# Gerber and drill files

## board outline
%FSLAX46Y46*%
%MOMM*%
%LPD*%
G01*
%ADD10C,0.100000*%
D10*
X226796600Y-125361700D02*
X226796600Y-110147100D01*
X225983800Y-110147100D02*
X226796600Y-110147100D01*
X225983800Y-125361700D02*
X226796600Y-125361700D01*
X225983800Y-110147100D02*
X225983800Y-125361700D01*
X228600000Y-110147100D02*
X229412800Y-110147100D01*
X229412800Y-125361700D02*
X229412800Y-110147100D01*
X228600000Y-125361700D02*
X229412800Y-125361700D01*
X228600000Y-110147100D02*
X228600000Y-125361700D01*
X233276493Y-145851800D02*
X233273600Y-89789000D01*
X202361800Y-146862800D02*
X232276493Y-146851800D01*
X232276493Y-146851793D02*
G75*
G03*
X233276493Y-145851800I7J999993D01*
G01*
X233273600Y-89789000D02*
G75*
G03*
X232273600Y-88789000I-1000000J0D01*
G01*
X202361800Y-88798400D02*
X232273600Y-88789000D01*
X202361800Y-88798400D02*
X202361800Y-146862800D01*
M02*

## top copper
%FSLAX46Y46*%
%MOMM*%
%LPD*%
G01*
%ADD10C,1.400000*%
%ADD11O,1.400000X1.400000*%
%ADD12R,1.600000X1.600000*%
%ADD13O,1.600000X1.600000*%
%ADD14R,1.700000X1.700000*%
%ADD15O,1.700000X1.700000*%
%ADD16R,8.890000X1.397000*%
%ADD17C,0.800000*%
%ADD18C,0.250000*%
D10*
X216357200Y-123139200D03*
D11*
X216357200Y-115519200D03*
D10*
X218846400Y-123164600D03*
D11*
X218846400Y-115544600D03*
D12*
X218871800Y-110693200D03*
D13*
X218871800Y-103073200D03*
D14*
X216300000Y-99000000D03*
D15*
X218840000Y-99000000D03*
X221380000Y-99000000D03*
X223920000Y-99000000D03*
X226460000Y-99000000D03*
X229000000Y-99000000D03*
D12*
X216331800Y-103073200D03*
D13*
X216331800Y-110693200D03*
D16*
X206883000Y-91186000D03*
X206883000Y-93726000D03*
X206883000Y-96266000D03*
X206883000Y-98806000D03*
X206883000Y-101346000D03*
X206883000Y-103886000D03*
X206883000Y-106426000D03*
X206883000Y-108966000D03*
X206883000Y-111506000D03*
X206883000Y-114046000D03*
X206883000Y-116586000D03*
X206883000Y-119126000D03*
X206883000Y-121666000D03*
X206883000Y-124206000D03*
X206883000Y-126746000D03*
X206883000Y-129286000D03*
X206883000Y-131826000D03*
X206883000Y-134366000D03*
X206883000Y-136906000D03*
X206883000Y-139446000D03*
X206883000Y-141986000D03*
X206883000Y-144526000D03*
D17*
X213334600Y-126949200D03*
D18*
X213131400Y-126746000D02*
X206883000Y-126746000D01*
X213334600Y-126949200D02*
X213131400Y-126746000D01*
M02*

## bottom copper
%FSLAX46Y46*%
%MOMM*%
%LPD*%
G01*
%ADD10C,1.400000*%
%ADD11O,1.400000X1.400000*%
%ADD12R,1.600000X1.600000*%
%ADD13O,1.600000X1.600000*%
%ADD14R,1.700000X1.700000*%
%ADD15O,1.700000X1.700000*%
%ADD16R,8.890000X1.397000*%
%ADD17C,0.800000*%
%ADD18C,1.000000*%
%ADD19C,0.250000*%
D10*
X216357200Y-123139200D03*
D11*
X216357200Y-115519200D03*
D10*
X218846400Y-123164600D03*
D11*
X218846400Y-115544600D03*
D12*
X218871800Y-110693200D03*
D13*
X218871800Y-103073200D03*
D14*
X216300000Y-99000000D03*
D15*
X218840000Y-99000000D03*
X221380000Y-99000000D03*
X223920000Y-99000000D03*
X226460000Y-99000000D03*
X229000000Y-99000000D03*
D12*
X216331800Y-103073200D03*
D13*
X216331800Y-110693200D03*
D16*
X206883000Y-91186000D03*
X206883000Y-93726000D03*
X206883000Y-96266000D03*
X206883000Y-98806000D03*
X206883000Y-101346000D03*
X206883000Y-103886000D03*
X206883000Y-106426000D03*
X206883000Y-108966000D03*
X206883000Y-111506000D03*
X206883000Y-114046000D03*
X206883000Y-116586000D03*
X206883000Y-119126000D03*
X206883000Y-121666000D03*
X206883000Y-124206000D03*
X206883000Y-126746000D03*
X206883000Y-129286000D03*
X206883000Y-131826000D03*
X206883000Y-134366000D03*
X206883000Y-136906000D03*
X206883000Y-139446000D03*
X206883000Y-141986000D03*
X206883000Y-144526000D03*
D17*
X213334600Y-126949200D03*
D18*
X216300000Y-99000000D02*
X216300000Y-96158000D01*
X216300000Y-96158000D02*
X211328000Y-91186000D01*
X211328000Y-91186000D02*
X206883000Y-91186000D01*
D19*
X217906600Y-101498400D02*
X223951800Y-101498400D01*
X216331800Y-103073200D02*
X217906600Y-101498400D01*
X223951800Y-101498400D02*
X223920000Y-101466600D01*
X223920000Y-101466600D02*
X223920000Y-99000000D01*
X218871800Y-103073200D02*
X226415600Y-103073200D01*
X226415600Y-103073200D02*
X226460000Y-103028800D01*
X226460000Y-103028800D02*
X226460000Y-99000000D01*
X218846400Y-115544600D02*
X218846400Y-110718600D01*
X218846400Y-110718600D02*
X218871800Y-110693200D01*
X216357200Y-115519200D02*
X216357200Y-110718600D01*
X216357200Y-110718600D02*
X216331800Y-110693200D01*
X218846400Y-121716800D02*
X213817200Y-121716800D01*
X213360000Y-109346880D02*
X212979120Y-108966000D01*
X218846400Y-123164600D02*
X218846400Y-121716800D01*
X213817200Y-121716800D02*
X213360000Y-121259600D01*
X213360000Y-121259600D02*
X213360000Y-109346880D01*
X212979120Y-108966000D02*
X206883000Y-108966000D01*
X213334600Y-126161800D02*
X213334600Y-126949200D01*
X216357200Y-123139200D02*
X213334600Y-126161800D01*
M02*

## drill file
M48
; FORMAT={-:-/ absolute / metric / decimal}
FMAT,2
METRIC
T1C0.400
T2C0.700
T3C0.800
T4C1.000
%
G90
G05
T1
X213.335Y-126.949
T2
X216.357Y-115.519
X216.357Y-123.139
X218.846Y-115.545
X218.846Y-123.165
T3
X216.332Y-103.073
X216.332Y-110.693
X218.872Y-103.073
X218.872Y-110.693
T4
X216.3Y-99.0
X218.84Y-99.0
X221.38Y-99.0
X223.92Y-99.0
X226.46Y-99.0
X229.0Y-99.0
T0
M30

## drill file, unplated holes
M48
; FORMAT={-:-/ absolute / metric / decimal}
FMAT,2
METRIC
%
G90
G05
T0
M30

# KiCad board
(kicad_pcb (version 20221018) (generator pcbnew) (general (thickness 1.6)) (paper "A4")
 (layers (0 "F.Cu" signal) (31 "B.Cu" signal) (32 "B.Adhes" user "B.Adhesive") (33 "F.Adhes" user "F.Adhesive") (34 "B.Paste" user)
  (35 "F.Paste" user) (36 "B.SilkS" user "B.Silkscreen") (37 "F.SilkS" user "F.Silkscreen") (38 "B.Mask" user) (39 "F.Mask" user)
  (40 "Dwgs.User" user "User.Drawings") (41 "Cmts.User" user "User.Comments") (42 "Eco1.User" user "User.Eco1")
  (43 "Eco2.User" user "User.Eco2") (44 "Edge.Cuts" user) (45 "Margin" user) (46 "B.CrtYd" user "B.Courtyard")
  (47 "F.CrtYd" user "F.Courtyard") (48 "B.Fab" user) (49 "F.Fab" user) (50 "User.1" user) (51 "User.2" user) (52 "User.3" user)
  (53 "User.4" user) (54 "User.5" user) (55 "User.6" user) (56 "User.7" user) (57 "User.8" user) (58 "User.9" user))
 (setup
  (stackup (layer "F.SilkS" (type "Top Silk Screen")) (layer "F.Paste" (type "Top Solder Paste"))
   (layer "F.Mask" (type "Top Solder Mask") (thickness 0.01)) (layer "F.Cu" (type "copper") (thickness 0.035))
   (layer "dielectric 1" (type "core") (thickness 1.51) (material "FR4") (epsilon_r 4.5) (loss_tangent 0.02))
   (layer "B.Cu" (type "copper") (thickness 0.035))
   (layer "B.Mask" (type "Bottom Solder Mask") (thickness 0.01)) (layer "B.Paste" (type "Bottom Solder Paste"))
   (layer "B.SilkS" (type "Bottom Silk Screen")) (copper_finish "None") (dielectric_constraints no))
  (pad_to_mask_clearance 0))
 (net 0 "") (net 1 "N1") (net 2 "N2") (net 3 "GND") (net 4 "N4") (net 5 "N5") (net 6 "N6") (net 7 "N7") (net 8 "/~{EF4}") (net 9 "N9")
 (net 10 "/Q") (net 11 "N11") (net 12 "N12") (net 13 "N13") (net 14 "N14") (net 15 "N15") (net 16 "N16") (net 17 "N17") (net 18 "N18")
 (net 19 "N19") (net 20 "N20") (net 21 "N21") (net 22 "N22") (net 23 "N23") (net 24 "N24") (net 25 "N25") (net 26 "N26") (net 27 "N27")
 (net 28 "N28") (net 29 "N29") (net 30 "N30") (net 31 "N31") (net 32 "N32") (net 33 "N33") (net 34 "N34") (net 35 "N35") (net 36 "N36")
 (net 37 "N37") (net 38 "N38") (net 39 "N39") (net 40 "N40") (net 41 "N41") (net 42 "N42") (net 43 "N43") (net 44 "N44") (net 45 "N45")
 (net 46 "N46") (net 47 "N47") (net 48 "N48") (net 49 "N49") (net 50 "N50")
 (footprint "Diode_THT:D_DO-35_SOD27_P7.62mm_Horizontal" (layer "F.Cu") (at 218.8718 110.6932 90)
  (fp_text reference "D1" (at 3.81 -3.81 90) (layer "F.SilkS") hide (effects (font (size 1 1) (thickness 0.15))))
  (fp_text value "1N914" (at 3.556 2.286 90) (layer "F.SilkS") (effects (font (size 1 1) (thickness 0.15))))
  (pad "1" thru_hole rect (at 0 0 90) (size 1.6 1.6) (drill 0.8) (layers "*.Cu" "*.Mask") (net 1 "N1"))
  (pad "2" thru_hole oval (at 7.62 0 90) (size 1.6 1.6) (drill 0.8) (layers "*.Cu" "*.Mask") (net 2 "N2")))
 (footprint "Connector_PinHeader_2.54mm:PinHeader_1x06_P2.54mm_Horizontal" (layer "F.Cu") (at 216.3 99 90)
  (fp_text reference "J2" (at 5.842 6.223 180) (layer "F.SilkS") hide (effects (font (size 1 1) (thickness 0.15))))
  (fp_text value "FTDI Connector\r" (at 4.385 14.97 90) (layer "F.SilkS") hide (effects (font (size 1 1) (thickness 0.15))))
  (pad "1" thru_hole rect (at 0 0 90) (size 1.7 1.7) (drill 1) (layers "*.Cu" "*.Mask") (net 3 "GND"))
  (pad "2" thru_hole oval (at 0 2.54 90) (size 1.7 1.7) (drill 1) (layers "*.Cu" "*.Mask") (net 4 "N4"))
  (pad "3" thru_hole oval (at 0 5.08 90) (size 1.7 1.7) (drill 1) (layers "*.Cu" "*.Mask") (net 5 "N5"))
  (pad "4" thru_hole oval (at 0 7.62 90) (size 1.7 1.7) (drill 1) (layers "*.Cu" "*.Mask") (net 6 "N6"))
  (pad "5" thru_hole oval (at 0 10.16 90) (size 1.7 1.7) (drill 1) (layers "*.Cu" "*.Mask") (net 2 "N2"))
  (pad "6" thru_hole oval (at 0 12.7 90) (size 1.7 1.7) (drill 1) (layers "*.Cu" "*.Mask") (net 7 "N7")))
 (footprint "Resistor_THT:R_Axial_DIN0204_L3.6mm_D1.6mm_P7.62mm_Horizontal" (layer "F.Cu") (at 216.3572 123.1392 90)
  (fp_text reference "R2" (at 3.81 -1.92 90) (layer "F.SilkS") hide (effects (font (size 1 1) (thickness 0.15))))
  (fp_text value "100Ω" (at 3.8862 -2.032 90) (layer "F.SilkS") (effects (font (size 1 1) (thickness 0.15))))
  (pad "1" thru_hole circle (at 0 0 90) (size 1.4 1.4) (drill 0.7) (layers "*.Cu" "*.Mask") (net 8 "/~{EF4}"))
  (pad "2" thru_hole oval (at 7.62 0 90) (size 1.4 1.4) (drill 0.7) (layers "*.Cu" "*.Mask") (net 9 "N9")))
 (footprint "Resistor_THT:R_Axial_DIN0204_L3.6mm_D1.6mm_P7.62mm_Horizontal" (layer "F.Cu") (at 218.8464 123.1646 90)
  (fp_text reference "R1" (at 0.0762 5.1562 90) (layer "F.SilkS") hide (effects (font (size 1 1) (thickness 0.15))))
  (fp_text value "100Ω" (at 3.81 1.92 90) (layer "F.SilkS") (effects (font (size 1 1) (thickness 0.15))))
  (pad "1" thru_hole circle (at 0 0 90) (size 1.4 1.4) (drill 0.7) (layers "*.Cu" "*.Mask") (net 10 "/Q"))
  (pad "2" thru_hole oval (at 7.62 0 90) (size 1.4 1.4) (drill 0.7) (layers "*.Cu" "*.Mask") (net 1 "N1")))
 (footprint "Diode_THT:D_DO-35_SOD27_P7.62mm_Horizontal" (layer "F.Cu") (at 216.3318 103.0732 -90)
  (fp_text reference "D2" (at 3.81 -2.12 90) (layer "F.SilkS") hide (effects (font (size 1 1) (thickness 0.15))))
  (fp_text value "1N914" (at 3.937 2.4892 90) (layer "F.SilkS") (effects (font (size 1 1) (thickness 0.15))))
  (pad "1" thru_hole rect (at 0 0 270) (size 1.6 1.6) (drill 0.8) (layers "*.Cu" "*.Mask") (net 6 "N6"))
  (pad "2" thru_hole oval (at 7.62 0 270) (size 1.6 1.6) (drill 0.8) (layers "*.Cu" "*.Mask") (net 9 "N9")))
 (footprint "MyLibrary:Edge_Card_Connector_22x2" (layer "F.Cu") (at 206.883 144.526 90)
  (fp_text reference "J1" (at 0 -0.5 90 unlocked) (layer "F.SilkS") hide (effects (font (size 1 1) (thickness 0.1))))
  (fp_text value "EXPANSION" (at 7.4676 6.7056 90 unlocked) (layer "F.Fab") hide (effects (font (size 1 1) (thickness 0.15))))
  (pad "1" connect rect (at 53.34 0 90) (size 1.397 8.89) (layers "B.Cu" "B.Mask") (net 3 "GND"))
  (pad "2" connect rect (at 53.34 0 90) (size 1.397 8.89) (layers "F.Cu" "F.Mask") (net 3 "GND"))
  (pad "3" connect rect (at 50.8 0 90) (size 1.397 8.89) (layers "B.Cu" "B.Mask") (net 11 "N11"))
  (pad "4" connect rect (at 50.8 0 90) (size 1.397 8.89) (layers "F.Cu" "F.Mask") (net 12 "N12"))
  (pad "5" connect rect (at 48.26 0 90) (size 1.397 8.89) (layers "B.Cu" "B.Mask") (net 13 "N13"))
  (pad "6" connect rect (at 48.26 0 90) (size 1.397 8.89) (layers "F.Cu" "F.Mask") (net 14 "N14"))
  (pad "7" connect rect (at 45.72 0 90) (size 1.397 8.89) (layers "B.Cu" "B.Mask") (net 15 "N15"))
  (pad "8" connect rect (at 45.72 0 90) (size 1.397 8.89) (layers "F.Cu" "F.Mask") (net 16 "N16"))
  (pad "9" connect rect (at 43.18 0 90) (size 1.397 8.89) (layers "B.Cu" "B.Mask") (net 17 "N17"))
  (pad "10" connect rect (at 43.18 0 90) (size 1.397 8.89) (layers "F.Cu" "F.Mask") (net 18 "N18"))
  (pad "11" connect rect (at 40.64 0 90) (size 1.397 8.89) (layers "B.Cu" "B.Mask") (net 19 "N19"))
  (pad "12" connect rect (at 40.64 0 90) (size 1.397 8.89) (layers "F.Cu" "F.Mask") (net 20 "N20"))
  (pad "13" connect rect (at 38.1 0 90) (size 1.397 8.89) (layers "B.Cu" "B.Mask") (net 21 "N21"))
  (pad "14" connect rect (at 38.1 0 90) (size 1.397 8.89) (layers "F.Cu" "F.Mask") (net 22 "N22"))
  (pad "15" connect rect (at 35.56 0 90) (size 1.397 8.89) (layers "B.Cu" "B.Mask") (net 10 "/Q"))
  (pad "16" connect rect (at 35.56 0 90) (size 1.397 8.89) (layers "F.Cu" "F.Mask") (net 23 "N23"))
  (pad "17" connect rect (at 33.02 0 90) (size 1.397 8.89) (layers "B.Cu" "B.Mask") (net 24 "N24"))
  (pad "18" connect rect (at 33.02 0 90) (size 1.397 8.89) (layers "F.Cu" "F.Mask") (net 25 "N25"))
  (pad "19" connect rect (at 30.48 0 90) (size 1.397 8.89) (layers "B.Cu" "B.Mask") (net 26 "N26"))
  (pad "20" connect rect (at 30.48 0 90) (size 1.397 8.89) (layers "F.Cu" "F.Mask") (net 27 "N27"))
  (pad "21" connect rect (at 27.94 0 90) (size 1.397 8.89) (layers "B.Cu" "B.Mask") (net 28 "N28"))
  (pad "22" connect rect (at 27.94 0 90) (size 1.397 8.89) (layers "F.Cu" "F.Mask") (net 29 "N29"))
  (pad "23" connect rect (at 25.4 0 90) (size 1.397 8.89) (layers "B.Cu" "B.Mask") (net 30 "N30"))
  (pad "24" connect rect (at 25.4 0 90) (size 1.397 8.89) (layers "F.Cu" "F.Mask") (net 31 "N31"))
  (pad "25" connect rect (at 22.86 0 90) (size 1.397 8.89) (layers "B.Cu" "B.Mask") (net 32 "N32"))
  (pad "26" connect rect (at 22.86 0 90) (size 1.397 8.89) (layers "F.Cu" "F.Mask") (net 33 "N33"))
  (pad "27" connect rect (at 20.32 0 90) (size 1.397 8.89) (layers "B.Cu" "B.Mask") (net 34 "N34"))
  (pad "28" connect rect (at 20.32 0 90) (size 1.397 8.89) (layers "F.Cu" "F.Mask") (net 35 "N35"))
  (pad "29" connect rect (at 17.78 0 90) (size 1.397 8.89) (layers "B.Cu" "B.Mask") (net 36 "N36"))
  (pad "30" connect rect (at 17.78 0 90) (size 1.397 8.89) (layers "F.Cu" "F.Mask") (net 8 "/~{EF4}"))
  (pad "31" connect rect (at 15.24 0 90) (size 1.397 8.89) (layers "B.Cu" "B.Mask") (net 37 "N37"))
  (pad "32" connect rect (at 15.24 0 90) (size 1.397 8.89) (layers "F.Cu" "F.Mask") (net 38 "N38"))
  (pad "33" connect rect (at 12.7 0 90) (size 1.397 8.89) (layers "B.Cu" "B.Mask") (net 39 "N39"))
  (pad "34" connect rect (at 12.7 0 90) (size 1.397 8.89) (layers "F.Cu" "F.Mask") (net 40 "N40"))
  (pad "35" connect rect (at 10.16 0 90) (size 1.397 8.89) (layers "B.Cu" "B.Mask") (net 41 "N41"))
  (pad "36" connect rect (at 10.16 0 90) (size 1.397 8.89) (layers "F.Cu" "F.Mask") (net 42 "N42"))
  (pad "37" connect rect (at 7.62 0 90) (size 1.397 8.89) (layers "B.Cu" "B.Mask") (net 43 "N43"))
  (pad "38" connect rect (at 7.62 0 90) (size 1.397 8.89) (layers "F.Cu" "F.Mask") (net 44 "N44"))
  (pad "39" connect rect (at 5.08 0 90) (size 1.397 8.89) (layers "B.Cu" "B.Mask") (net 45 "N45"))
  (pad "40" connect rect (at 5.08 0 90) (size 1.397 8.89) (layers "F.Cu" "F.Mask") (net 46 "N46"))
  (pad "41" connect rect (at 2.54 0 90) (size 1.397 8.89) (layers "B.Cu" "B.Mask") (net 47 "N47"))
  (pad "42" connect rect (at 2.54 0 90) (size 1.397 8.89) (layers "F.Cu" "F.Mask") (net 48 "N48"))
  (pad "43" connect rect (at 0 0 90) (size 1.397 8.89) (layers "B.Cu" "B.Mask") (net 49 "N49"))
  (pad "44" connect rect (at 0 0 90) (size 1.397 8.89) (layers "F.Cu" "F.Mask") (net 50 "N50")))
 (gr_line (start 233.276493 145.8518) (end 233.2736 89.789) (stroke (width 0.1) (type default)) (layer "Edge.Cuts"))
 (gr_line (start 202.3618 146.8628) (end 232.276493 146.8518) (stroke (width 0.1) (type default)) (layer "Edge.Cuts"))
 (gr_arc (start 233.276493 145.8518) (mid 232.983599 146.558904) (end 232.276493 146.8518) (stroke (width 0.1) (type default))
  (layer "Edge.Cuts"))
 (gr_line (start 228.6 125.3617) (end 229.4128 125.3617) (stroke (width 0.1) (type default)) (layer "Edge.Cuts"))
 (gr_line (start 229.4128 125.3617) (end 229.4128 110.1471) (stroke (width 0.1) (type default)) (layer "Edge.Cuts"))
 (gr_line (start 225.9838 125.3617) (end 226.7966 125.3617) (stroke (width 0.1) (type default)) (layer "Edge.Cuts"))
 (gr_arc (start 232.2736 88.789) (mid 232.980707 89.081893) (end 233.2736 89.789) (stroke (width 0.1) (type default)) (layer "Edge.Cuts"))
 (gr_line (start 225.9838 110.1471) (end 225.9838 125.3617) (stroke (width 0.1) (type default)) (layer "Edge.Cuts"))
 (gr_line (start 228.6 110.1471) (end 228.6 125.3617) (stroke (width 0.1) (type default)) (layer "Edge.Cuts"))
 (gr_line (start 202.3618 88.7984) (end 232.2736 88.789) (stroke (width 0.1) (type default)) (layer "Edge.Cuts"))
 (gr_line (start 228.6 110.1471) (end 229.4128 110.1471) (stroke (width 0.1) (type default)) (layer "Edge.Cuts"))
 (gr_line (start 202.3618 88.7984) (end 202.3618 146.8628) (stroke (width 0.1) (type default)) (layer "Edge.Cuts"))
 (gr_line (start 225.9838 110.1471) (end 226.7966 110.1471) (stroke (width 0.1) (type default)) (layer "Edge.Cuts"))
 (gr_line (start 226.7966 125.3617) (end 226.7966 110.1471) (stroke (width 0.1) (type default)) (layer "Edge.Cuts"))
 (segment (start 218.8464 110.7186) (end 218.8718 110.6932) (width 0.25) (layer "B.Cu") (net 1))
 (segment (start 218.8464 115.5446) (end 218.8464 110.7186) (width 0.25) (layer "B.Cu") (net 1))
 (segment (start 213.3346 126.9492) (end 213.1314 126.746) (width 0.25) (layer "F.Cu") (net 8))
 (segment (start 213.1314 126.746) (end 206.883 126.746) (width 0.25) (layer "F.Cu") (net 8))
 (via (at 213.3346 126.9492) (size 0.8) (drill 0.4) (layers "F.Cu" "B.Cu") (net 8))
 (segment (start 216.3572 123.1392) (end 213.3346 126.1618) (width 0.25) (layer "B.Cu") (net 8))
 (segment (start 213.3346 126.1618) (end 213.3346 126.9492) (width 0.25) (layer "B.Cu") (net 8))
 (segment (start 211.328 91.186) (end 206.883 91.186) (width 1) (layer "B.Cu") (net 3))
 (segment (start 216.3 99) (end 216.3 96.158) (width 1) (layer "B.Cu") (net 3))
 (segment (start 216.3 96.158) (end 211.328 91.186) (width 1) (layer "B.Cu") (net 3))
 (segment (start 213.36 121.2596) (end 213.36 109.34688) (width 0.25) (layer "B.Cu") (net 10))
 (segment (start 213.8172 121.7168) (end 213.36 121.2596) (width 0.25) (layer "B.Cu") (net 10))
 (segment (start 218.8464 123.1646) (end 218.8464 121.7168) (width 0.25) (layer "B.Cu") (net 10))
 (segment (start 212.97912 108.966) (end 206.883 108.966) (width 0.25) (layer "B.Cu") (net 10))
 (segment (start 213.36 109.34688) (end 212.97912 108.966) (width 0.25) (layer "B.Cu") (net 10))
 (segment (start 218.8464 121.7168) (end 213.8172 121.7168) (width 0.25) (layer "B.Cu") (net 10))
 (segment (start 218.8718 103.0732) (end 226.4156 103.0732) (width 0.25) (layer "B.Cu") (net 2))
 (segment (start 226.46 103.0288) (end 226.46 99) (width 0.25) (layer "B.Cu") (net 2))
 (segment (start 226.4156 103.0732) (end 226.46 103.0288) (width 0.25) (layer "B.Cu") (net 2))
 (segment (start 223.92 101.4666) (end 223.92 99) (width 0.25) (layer "B.Cu") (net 6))
 (segment (start 217.9066 101.4984) (end 223.9518 101.4984) (width 0.25) (layer "B.Cu") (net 6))
 (segment (start 223.9518 101.4984) (end 223.92 101.4666) (width 0.25) (layer "B.Cu") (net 6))
 (segment (start 216.3318 103.0732) (end 217.9066 101.4984) (width 0.25) (layer "B.Cu") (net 6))
 (segment (start 216.3572 110.7186) (end 216.3318 110.6932) (width 0.25) (layer "B.Cu") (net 9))
 (segment (start 216.3572 115.5192) (end 216.3572 110.7186) (width 0.25) (layer "B.Cu") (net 9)))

